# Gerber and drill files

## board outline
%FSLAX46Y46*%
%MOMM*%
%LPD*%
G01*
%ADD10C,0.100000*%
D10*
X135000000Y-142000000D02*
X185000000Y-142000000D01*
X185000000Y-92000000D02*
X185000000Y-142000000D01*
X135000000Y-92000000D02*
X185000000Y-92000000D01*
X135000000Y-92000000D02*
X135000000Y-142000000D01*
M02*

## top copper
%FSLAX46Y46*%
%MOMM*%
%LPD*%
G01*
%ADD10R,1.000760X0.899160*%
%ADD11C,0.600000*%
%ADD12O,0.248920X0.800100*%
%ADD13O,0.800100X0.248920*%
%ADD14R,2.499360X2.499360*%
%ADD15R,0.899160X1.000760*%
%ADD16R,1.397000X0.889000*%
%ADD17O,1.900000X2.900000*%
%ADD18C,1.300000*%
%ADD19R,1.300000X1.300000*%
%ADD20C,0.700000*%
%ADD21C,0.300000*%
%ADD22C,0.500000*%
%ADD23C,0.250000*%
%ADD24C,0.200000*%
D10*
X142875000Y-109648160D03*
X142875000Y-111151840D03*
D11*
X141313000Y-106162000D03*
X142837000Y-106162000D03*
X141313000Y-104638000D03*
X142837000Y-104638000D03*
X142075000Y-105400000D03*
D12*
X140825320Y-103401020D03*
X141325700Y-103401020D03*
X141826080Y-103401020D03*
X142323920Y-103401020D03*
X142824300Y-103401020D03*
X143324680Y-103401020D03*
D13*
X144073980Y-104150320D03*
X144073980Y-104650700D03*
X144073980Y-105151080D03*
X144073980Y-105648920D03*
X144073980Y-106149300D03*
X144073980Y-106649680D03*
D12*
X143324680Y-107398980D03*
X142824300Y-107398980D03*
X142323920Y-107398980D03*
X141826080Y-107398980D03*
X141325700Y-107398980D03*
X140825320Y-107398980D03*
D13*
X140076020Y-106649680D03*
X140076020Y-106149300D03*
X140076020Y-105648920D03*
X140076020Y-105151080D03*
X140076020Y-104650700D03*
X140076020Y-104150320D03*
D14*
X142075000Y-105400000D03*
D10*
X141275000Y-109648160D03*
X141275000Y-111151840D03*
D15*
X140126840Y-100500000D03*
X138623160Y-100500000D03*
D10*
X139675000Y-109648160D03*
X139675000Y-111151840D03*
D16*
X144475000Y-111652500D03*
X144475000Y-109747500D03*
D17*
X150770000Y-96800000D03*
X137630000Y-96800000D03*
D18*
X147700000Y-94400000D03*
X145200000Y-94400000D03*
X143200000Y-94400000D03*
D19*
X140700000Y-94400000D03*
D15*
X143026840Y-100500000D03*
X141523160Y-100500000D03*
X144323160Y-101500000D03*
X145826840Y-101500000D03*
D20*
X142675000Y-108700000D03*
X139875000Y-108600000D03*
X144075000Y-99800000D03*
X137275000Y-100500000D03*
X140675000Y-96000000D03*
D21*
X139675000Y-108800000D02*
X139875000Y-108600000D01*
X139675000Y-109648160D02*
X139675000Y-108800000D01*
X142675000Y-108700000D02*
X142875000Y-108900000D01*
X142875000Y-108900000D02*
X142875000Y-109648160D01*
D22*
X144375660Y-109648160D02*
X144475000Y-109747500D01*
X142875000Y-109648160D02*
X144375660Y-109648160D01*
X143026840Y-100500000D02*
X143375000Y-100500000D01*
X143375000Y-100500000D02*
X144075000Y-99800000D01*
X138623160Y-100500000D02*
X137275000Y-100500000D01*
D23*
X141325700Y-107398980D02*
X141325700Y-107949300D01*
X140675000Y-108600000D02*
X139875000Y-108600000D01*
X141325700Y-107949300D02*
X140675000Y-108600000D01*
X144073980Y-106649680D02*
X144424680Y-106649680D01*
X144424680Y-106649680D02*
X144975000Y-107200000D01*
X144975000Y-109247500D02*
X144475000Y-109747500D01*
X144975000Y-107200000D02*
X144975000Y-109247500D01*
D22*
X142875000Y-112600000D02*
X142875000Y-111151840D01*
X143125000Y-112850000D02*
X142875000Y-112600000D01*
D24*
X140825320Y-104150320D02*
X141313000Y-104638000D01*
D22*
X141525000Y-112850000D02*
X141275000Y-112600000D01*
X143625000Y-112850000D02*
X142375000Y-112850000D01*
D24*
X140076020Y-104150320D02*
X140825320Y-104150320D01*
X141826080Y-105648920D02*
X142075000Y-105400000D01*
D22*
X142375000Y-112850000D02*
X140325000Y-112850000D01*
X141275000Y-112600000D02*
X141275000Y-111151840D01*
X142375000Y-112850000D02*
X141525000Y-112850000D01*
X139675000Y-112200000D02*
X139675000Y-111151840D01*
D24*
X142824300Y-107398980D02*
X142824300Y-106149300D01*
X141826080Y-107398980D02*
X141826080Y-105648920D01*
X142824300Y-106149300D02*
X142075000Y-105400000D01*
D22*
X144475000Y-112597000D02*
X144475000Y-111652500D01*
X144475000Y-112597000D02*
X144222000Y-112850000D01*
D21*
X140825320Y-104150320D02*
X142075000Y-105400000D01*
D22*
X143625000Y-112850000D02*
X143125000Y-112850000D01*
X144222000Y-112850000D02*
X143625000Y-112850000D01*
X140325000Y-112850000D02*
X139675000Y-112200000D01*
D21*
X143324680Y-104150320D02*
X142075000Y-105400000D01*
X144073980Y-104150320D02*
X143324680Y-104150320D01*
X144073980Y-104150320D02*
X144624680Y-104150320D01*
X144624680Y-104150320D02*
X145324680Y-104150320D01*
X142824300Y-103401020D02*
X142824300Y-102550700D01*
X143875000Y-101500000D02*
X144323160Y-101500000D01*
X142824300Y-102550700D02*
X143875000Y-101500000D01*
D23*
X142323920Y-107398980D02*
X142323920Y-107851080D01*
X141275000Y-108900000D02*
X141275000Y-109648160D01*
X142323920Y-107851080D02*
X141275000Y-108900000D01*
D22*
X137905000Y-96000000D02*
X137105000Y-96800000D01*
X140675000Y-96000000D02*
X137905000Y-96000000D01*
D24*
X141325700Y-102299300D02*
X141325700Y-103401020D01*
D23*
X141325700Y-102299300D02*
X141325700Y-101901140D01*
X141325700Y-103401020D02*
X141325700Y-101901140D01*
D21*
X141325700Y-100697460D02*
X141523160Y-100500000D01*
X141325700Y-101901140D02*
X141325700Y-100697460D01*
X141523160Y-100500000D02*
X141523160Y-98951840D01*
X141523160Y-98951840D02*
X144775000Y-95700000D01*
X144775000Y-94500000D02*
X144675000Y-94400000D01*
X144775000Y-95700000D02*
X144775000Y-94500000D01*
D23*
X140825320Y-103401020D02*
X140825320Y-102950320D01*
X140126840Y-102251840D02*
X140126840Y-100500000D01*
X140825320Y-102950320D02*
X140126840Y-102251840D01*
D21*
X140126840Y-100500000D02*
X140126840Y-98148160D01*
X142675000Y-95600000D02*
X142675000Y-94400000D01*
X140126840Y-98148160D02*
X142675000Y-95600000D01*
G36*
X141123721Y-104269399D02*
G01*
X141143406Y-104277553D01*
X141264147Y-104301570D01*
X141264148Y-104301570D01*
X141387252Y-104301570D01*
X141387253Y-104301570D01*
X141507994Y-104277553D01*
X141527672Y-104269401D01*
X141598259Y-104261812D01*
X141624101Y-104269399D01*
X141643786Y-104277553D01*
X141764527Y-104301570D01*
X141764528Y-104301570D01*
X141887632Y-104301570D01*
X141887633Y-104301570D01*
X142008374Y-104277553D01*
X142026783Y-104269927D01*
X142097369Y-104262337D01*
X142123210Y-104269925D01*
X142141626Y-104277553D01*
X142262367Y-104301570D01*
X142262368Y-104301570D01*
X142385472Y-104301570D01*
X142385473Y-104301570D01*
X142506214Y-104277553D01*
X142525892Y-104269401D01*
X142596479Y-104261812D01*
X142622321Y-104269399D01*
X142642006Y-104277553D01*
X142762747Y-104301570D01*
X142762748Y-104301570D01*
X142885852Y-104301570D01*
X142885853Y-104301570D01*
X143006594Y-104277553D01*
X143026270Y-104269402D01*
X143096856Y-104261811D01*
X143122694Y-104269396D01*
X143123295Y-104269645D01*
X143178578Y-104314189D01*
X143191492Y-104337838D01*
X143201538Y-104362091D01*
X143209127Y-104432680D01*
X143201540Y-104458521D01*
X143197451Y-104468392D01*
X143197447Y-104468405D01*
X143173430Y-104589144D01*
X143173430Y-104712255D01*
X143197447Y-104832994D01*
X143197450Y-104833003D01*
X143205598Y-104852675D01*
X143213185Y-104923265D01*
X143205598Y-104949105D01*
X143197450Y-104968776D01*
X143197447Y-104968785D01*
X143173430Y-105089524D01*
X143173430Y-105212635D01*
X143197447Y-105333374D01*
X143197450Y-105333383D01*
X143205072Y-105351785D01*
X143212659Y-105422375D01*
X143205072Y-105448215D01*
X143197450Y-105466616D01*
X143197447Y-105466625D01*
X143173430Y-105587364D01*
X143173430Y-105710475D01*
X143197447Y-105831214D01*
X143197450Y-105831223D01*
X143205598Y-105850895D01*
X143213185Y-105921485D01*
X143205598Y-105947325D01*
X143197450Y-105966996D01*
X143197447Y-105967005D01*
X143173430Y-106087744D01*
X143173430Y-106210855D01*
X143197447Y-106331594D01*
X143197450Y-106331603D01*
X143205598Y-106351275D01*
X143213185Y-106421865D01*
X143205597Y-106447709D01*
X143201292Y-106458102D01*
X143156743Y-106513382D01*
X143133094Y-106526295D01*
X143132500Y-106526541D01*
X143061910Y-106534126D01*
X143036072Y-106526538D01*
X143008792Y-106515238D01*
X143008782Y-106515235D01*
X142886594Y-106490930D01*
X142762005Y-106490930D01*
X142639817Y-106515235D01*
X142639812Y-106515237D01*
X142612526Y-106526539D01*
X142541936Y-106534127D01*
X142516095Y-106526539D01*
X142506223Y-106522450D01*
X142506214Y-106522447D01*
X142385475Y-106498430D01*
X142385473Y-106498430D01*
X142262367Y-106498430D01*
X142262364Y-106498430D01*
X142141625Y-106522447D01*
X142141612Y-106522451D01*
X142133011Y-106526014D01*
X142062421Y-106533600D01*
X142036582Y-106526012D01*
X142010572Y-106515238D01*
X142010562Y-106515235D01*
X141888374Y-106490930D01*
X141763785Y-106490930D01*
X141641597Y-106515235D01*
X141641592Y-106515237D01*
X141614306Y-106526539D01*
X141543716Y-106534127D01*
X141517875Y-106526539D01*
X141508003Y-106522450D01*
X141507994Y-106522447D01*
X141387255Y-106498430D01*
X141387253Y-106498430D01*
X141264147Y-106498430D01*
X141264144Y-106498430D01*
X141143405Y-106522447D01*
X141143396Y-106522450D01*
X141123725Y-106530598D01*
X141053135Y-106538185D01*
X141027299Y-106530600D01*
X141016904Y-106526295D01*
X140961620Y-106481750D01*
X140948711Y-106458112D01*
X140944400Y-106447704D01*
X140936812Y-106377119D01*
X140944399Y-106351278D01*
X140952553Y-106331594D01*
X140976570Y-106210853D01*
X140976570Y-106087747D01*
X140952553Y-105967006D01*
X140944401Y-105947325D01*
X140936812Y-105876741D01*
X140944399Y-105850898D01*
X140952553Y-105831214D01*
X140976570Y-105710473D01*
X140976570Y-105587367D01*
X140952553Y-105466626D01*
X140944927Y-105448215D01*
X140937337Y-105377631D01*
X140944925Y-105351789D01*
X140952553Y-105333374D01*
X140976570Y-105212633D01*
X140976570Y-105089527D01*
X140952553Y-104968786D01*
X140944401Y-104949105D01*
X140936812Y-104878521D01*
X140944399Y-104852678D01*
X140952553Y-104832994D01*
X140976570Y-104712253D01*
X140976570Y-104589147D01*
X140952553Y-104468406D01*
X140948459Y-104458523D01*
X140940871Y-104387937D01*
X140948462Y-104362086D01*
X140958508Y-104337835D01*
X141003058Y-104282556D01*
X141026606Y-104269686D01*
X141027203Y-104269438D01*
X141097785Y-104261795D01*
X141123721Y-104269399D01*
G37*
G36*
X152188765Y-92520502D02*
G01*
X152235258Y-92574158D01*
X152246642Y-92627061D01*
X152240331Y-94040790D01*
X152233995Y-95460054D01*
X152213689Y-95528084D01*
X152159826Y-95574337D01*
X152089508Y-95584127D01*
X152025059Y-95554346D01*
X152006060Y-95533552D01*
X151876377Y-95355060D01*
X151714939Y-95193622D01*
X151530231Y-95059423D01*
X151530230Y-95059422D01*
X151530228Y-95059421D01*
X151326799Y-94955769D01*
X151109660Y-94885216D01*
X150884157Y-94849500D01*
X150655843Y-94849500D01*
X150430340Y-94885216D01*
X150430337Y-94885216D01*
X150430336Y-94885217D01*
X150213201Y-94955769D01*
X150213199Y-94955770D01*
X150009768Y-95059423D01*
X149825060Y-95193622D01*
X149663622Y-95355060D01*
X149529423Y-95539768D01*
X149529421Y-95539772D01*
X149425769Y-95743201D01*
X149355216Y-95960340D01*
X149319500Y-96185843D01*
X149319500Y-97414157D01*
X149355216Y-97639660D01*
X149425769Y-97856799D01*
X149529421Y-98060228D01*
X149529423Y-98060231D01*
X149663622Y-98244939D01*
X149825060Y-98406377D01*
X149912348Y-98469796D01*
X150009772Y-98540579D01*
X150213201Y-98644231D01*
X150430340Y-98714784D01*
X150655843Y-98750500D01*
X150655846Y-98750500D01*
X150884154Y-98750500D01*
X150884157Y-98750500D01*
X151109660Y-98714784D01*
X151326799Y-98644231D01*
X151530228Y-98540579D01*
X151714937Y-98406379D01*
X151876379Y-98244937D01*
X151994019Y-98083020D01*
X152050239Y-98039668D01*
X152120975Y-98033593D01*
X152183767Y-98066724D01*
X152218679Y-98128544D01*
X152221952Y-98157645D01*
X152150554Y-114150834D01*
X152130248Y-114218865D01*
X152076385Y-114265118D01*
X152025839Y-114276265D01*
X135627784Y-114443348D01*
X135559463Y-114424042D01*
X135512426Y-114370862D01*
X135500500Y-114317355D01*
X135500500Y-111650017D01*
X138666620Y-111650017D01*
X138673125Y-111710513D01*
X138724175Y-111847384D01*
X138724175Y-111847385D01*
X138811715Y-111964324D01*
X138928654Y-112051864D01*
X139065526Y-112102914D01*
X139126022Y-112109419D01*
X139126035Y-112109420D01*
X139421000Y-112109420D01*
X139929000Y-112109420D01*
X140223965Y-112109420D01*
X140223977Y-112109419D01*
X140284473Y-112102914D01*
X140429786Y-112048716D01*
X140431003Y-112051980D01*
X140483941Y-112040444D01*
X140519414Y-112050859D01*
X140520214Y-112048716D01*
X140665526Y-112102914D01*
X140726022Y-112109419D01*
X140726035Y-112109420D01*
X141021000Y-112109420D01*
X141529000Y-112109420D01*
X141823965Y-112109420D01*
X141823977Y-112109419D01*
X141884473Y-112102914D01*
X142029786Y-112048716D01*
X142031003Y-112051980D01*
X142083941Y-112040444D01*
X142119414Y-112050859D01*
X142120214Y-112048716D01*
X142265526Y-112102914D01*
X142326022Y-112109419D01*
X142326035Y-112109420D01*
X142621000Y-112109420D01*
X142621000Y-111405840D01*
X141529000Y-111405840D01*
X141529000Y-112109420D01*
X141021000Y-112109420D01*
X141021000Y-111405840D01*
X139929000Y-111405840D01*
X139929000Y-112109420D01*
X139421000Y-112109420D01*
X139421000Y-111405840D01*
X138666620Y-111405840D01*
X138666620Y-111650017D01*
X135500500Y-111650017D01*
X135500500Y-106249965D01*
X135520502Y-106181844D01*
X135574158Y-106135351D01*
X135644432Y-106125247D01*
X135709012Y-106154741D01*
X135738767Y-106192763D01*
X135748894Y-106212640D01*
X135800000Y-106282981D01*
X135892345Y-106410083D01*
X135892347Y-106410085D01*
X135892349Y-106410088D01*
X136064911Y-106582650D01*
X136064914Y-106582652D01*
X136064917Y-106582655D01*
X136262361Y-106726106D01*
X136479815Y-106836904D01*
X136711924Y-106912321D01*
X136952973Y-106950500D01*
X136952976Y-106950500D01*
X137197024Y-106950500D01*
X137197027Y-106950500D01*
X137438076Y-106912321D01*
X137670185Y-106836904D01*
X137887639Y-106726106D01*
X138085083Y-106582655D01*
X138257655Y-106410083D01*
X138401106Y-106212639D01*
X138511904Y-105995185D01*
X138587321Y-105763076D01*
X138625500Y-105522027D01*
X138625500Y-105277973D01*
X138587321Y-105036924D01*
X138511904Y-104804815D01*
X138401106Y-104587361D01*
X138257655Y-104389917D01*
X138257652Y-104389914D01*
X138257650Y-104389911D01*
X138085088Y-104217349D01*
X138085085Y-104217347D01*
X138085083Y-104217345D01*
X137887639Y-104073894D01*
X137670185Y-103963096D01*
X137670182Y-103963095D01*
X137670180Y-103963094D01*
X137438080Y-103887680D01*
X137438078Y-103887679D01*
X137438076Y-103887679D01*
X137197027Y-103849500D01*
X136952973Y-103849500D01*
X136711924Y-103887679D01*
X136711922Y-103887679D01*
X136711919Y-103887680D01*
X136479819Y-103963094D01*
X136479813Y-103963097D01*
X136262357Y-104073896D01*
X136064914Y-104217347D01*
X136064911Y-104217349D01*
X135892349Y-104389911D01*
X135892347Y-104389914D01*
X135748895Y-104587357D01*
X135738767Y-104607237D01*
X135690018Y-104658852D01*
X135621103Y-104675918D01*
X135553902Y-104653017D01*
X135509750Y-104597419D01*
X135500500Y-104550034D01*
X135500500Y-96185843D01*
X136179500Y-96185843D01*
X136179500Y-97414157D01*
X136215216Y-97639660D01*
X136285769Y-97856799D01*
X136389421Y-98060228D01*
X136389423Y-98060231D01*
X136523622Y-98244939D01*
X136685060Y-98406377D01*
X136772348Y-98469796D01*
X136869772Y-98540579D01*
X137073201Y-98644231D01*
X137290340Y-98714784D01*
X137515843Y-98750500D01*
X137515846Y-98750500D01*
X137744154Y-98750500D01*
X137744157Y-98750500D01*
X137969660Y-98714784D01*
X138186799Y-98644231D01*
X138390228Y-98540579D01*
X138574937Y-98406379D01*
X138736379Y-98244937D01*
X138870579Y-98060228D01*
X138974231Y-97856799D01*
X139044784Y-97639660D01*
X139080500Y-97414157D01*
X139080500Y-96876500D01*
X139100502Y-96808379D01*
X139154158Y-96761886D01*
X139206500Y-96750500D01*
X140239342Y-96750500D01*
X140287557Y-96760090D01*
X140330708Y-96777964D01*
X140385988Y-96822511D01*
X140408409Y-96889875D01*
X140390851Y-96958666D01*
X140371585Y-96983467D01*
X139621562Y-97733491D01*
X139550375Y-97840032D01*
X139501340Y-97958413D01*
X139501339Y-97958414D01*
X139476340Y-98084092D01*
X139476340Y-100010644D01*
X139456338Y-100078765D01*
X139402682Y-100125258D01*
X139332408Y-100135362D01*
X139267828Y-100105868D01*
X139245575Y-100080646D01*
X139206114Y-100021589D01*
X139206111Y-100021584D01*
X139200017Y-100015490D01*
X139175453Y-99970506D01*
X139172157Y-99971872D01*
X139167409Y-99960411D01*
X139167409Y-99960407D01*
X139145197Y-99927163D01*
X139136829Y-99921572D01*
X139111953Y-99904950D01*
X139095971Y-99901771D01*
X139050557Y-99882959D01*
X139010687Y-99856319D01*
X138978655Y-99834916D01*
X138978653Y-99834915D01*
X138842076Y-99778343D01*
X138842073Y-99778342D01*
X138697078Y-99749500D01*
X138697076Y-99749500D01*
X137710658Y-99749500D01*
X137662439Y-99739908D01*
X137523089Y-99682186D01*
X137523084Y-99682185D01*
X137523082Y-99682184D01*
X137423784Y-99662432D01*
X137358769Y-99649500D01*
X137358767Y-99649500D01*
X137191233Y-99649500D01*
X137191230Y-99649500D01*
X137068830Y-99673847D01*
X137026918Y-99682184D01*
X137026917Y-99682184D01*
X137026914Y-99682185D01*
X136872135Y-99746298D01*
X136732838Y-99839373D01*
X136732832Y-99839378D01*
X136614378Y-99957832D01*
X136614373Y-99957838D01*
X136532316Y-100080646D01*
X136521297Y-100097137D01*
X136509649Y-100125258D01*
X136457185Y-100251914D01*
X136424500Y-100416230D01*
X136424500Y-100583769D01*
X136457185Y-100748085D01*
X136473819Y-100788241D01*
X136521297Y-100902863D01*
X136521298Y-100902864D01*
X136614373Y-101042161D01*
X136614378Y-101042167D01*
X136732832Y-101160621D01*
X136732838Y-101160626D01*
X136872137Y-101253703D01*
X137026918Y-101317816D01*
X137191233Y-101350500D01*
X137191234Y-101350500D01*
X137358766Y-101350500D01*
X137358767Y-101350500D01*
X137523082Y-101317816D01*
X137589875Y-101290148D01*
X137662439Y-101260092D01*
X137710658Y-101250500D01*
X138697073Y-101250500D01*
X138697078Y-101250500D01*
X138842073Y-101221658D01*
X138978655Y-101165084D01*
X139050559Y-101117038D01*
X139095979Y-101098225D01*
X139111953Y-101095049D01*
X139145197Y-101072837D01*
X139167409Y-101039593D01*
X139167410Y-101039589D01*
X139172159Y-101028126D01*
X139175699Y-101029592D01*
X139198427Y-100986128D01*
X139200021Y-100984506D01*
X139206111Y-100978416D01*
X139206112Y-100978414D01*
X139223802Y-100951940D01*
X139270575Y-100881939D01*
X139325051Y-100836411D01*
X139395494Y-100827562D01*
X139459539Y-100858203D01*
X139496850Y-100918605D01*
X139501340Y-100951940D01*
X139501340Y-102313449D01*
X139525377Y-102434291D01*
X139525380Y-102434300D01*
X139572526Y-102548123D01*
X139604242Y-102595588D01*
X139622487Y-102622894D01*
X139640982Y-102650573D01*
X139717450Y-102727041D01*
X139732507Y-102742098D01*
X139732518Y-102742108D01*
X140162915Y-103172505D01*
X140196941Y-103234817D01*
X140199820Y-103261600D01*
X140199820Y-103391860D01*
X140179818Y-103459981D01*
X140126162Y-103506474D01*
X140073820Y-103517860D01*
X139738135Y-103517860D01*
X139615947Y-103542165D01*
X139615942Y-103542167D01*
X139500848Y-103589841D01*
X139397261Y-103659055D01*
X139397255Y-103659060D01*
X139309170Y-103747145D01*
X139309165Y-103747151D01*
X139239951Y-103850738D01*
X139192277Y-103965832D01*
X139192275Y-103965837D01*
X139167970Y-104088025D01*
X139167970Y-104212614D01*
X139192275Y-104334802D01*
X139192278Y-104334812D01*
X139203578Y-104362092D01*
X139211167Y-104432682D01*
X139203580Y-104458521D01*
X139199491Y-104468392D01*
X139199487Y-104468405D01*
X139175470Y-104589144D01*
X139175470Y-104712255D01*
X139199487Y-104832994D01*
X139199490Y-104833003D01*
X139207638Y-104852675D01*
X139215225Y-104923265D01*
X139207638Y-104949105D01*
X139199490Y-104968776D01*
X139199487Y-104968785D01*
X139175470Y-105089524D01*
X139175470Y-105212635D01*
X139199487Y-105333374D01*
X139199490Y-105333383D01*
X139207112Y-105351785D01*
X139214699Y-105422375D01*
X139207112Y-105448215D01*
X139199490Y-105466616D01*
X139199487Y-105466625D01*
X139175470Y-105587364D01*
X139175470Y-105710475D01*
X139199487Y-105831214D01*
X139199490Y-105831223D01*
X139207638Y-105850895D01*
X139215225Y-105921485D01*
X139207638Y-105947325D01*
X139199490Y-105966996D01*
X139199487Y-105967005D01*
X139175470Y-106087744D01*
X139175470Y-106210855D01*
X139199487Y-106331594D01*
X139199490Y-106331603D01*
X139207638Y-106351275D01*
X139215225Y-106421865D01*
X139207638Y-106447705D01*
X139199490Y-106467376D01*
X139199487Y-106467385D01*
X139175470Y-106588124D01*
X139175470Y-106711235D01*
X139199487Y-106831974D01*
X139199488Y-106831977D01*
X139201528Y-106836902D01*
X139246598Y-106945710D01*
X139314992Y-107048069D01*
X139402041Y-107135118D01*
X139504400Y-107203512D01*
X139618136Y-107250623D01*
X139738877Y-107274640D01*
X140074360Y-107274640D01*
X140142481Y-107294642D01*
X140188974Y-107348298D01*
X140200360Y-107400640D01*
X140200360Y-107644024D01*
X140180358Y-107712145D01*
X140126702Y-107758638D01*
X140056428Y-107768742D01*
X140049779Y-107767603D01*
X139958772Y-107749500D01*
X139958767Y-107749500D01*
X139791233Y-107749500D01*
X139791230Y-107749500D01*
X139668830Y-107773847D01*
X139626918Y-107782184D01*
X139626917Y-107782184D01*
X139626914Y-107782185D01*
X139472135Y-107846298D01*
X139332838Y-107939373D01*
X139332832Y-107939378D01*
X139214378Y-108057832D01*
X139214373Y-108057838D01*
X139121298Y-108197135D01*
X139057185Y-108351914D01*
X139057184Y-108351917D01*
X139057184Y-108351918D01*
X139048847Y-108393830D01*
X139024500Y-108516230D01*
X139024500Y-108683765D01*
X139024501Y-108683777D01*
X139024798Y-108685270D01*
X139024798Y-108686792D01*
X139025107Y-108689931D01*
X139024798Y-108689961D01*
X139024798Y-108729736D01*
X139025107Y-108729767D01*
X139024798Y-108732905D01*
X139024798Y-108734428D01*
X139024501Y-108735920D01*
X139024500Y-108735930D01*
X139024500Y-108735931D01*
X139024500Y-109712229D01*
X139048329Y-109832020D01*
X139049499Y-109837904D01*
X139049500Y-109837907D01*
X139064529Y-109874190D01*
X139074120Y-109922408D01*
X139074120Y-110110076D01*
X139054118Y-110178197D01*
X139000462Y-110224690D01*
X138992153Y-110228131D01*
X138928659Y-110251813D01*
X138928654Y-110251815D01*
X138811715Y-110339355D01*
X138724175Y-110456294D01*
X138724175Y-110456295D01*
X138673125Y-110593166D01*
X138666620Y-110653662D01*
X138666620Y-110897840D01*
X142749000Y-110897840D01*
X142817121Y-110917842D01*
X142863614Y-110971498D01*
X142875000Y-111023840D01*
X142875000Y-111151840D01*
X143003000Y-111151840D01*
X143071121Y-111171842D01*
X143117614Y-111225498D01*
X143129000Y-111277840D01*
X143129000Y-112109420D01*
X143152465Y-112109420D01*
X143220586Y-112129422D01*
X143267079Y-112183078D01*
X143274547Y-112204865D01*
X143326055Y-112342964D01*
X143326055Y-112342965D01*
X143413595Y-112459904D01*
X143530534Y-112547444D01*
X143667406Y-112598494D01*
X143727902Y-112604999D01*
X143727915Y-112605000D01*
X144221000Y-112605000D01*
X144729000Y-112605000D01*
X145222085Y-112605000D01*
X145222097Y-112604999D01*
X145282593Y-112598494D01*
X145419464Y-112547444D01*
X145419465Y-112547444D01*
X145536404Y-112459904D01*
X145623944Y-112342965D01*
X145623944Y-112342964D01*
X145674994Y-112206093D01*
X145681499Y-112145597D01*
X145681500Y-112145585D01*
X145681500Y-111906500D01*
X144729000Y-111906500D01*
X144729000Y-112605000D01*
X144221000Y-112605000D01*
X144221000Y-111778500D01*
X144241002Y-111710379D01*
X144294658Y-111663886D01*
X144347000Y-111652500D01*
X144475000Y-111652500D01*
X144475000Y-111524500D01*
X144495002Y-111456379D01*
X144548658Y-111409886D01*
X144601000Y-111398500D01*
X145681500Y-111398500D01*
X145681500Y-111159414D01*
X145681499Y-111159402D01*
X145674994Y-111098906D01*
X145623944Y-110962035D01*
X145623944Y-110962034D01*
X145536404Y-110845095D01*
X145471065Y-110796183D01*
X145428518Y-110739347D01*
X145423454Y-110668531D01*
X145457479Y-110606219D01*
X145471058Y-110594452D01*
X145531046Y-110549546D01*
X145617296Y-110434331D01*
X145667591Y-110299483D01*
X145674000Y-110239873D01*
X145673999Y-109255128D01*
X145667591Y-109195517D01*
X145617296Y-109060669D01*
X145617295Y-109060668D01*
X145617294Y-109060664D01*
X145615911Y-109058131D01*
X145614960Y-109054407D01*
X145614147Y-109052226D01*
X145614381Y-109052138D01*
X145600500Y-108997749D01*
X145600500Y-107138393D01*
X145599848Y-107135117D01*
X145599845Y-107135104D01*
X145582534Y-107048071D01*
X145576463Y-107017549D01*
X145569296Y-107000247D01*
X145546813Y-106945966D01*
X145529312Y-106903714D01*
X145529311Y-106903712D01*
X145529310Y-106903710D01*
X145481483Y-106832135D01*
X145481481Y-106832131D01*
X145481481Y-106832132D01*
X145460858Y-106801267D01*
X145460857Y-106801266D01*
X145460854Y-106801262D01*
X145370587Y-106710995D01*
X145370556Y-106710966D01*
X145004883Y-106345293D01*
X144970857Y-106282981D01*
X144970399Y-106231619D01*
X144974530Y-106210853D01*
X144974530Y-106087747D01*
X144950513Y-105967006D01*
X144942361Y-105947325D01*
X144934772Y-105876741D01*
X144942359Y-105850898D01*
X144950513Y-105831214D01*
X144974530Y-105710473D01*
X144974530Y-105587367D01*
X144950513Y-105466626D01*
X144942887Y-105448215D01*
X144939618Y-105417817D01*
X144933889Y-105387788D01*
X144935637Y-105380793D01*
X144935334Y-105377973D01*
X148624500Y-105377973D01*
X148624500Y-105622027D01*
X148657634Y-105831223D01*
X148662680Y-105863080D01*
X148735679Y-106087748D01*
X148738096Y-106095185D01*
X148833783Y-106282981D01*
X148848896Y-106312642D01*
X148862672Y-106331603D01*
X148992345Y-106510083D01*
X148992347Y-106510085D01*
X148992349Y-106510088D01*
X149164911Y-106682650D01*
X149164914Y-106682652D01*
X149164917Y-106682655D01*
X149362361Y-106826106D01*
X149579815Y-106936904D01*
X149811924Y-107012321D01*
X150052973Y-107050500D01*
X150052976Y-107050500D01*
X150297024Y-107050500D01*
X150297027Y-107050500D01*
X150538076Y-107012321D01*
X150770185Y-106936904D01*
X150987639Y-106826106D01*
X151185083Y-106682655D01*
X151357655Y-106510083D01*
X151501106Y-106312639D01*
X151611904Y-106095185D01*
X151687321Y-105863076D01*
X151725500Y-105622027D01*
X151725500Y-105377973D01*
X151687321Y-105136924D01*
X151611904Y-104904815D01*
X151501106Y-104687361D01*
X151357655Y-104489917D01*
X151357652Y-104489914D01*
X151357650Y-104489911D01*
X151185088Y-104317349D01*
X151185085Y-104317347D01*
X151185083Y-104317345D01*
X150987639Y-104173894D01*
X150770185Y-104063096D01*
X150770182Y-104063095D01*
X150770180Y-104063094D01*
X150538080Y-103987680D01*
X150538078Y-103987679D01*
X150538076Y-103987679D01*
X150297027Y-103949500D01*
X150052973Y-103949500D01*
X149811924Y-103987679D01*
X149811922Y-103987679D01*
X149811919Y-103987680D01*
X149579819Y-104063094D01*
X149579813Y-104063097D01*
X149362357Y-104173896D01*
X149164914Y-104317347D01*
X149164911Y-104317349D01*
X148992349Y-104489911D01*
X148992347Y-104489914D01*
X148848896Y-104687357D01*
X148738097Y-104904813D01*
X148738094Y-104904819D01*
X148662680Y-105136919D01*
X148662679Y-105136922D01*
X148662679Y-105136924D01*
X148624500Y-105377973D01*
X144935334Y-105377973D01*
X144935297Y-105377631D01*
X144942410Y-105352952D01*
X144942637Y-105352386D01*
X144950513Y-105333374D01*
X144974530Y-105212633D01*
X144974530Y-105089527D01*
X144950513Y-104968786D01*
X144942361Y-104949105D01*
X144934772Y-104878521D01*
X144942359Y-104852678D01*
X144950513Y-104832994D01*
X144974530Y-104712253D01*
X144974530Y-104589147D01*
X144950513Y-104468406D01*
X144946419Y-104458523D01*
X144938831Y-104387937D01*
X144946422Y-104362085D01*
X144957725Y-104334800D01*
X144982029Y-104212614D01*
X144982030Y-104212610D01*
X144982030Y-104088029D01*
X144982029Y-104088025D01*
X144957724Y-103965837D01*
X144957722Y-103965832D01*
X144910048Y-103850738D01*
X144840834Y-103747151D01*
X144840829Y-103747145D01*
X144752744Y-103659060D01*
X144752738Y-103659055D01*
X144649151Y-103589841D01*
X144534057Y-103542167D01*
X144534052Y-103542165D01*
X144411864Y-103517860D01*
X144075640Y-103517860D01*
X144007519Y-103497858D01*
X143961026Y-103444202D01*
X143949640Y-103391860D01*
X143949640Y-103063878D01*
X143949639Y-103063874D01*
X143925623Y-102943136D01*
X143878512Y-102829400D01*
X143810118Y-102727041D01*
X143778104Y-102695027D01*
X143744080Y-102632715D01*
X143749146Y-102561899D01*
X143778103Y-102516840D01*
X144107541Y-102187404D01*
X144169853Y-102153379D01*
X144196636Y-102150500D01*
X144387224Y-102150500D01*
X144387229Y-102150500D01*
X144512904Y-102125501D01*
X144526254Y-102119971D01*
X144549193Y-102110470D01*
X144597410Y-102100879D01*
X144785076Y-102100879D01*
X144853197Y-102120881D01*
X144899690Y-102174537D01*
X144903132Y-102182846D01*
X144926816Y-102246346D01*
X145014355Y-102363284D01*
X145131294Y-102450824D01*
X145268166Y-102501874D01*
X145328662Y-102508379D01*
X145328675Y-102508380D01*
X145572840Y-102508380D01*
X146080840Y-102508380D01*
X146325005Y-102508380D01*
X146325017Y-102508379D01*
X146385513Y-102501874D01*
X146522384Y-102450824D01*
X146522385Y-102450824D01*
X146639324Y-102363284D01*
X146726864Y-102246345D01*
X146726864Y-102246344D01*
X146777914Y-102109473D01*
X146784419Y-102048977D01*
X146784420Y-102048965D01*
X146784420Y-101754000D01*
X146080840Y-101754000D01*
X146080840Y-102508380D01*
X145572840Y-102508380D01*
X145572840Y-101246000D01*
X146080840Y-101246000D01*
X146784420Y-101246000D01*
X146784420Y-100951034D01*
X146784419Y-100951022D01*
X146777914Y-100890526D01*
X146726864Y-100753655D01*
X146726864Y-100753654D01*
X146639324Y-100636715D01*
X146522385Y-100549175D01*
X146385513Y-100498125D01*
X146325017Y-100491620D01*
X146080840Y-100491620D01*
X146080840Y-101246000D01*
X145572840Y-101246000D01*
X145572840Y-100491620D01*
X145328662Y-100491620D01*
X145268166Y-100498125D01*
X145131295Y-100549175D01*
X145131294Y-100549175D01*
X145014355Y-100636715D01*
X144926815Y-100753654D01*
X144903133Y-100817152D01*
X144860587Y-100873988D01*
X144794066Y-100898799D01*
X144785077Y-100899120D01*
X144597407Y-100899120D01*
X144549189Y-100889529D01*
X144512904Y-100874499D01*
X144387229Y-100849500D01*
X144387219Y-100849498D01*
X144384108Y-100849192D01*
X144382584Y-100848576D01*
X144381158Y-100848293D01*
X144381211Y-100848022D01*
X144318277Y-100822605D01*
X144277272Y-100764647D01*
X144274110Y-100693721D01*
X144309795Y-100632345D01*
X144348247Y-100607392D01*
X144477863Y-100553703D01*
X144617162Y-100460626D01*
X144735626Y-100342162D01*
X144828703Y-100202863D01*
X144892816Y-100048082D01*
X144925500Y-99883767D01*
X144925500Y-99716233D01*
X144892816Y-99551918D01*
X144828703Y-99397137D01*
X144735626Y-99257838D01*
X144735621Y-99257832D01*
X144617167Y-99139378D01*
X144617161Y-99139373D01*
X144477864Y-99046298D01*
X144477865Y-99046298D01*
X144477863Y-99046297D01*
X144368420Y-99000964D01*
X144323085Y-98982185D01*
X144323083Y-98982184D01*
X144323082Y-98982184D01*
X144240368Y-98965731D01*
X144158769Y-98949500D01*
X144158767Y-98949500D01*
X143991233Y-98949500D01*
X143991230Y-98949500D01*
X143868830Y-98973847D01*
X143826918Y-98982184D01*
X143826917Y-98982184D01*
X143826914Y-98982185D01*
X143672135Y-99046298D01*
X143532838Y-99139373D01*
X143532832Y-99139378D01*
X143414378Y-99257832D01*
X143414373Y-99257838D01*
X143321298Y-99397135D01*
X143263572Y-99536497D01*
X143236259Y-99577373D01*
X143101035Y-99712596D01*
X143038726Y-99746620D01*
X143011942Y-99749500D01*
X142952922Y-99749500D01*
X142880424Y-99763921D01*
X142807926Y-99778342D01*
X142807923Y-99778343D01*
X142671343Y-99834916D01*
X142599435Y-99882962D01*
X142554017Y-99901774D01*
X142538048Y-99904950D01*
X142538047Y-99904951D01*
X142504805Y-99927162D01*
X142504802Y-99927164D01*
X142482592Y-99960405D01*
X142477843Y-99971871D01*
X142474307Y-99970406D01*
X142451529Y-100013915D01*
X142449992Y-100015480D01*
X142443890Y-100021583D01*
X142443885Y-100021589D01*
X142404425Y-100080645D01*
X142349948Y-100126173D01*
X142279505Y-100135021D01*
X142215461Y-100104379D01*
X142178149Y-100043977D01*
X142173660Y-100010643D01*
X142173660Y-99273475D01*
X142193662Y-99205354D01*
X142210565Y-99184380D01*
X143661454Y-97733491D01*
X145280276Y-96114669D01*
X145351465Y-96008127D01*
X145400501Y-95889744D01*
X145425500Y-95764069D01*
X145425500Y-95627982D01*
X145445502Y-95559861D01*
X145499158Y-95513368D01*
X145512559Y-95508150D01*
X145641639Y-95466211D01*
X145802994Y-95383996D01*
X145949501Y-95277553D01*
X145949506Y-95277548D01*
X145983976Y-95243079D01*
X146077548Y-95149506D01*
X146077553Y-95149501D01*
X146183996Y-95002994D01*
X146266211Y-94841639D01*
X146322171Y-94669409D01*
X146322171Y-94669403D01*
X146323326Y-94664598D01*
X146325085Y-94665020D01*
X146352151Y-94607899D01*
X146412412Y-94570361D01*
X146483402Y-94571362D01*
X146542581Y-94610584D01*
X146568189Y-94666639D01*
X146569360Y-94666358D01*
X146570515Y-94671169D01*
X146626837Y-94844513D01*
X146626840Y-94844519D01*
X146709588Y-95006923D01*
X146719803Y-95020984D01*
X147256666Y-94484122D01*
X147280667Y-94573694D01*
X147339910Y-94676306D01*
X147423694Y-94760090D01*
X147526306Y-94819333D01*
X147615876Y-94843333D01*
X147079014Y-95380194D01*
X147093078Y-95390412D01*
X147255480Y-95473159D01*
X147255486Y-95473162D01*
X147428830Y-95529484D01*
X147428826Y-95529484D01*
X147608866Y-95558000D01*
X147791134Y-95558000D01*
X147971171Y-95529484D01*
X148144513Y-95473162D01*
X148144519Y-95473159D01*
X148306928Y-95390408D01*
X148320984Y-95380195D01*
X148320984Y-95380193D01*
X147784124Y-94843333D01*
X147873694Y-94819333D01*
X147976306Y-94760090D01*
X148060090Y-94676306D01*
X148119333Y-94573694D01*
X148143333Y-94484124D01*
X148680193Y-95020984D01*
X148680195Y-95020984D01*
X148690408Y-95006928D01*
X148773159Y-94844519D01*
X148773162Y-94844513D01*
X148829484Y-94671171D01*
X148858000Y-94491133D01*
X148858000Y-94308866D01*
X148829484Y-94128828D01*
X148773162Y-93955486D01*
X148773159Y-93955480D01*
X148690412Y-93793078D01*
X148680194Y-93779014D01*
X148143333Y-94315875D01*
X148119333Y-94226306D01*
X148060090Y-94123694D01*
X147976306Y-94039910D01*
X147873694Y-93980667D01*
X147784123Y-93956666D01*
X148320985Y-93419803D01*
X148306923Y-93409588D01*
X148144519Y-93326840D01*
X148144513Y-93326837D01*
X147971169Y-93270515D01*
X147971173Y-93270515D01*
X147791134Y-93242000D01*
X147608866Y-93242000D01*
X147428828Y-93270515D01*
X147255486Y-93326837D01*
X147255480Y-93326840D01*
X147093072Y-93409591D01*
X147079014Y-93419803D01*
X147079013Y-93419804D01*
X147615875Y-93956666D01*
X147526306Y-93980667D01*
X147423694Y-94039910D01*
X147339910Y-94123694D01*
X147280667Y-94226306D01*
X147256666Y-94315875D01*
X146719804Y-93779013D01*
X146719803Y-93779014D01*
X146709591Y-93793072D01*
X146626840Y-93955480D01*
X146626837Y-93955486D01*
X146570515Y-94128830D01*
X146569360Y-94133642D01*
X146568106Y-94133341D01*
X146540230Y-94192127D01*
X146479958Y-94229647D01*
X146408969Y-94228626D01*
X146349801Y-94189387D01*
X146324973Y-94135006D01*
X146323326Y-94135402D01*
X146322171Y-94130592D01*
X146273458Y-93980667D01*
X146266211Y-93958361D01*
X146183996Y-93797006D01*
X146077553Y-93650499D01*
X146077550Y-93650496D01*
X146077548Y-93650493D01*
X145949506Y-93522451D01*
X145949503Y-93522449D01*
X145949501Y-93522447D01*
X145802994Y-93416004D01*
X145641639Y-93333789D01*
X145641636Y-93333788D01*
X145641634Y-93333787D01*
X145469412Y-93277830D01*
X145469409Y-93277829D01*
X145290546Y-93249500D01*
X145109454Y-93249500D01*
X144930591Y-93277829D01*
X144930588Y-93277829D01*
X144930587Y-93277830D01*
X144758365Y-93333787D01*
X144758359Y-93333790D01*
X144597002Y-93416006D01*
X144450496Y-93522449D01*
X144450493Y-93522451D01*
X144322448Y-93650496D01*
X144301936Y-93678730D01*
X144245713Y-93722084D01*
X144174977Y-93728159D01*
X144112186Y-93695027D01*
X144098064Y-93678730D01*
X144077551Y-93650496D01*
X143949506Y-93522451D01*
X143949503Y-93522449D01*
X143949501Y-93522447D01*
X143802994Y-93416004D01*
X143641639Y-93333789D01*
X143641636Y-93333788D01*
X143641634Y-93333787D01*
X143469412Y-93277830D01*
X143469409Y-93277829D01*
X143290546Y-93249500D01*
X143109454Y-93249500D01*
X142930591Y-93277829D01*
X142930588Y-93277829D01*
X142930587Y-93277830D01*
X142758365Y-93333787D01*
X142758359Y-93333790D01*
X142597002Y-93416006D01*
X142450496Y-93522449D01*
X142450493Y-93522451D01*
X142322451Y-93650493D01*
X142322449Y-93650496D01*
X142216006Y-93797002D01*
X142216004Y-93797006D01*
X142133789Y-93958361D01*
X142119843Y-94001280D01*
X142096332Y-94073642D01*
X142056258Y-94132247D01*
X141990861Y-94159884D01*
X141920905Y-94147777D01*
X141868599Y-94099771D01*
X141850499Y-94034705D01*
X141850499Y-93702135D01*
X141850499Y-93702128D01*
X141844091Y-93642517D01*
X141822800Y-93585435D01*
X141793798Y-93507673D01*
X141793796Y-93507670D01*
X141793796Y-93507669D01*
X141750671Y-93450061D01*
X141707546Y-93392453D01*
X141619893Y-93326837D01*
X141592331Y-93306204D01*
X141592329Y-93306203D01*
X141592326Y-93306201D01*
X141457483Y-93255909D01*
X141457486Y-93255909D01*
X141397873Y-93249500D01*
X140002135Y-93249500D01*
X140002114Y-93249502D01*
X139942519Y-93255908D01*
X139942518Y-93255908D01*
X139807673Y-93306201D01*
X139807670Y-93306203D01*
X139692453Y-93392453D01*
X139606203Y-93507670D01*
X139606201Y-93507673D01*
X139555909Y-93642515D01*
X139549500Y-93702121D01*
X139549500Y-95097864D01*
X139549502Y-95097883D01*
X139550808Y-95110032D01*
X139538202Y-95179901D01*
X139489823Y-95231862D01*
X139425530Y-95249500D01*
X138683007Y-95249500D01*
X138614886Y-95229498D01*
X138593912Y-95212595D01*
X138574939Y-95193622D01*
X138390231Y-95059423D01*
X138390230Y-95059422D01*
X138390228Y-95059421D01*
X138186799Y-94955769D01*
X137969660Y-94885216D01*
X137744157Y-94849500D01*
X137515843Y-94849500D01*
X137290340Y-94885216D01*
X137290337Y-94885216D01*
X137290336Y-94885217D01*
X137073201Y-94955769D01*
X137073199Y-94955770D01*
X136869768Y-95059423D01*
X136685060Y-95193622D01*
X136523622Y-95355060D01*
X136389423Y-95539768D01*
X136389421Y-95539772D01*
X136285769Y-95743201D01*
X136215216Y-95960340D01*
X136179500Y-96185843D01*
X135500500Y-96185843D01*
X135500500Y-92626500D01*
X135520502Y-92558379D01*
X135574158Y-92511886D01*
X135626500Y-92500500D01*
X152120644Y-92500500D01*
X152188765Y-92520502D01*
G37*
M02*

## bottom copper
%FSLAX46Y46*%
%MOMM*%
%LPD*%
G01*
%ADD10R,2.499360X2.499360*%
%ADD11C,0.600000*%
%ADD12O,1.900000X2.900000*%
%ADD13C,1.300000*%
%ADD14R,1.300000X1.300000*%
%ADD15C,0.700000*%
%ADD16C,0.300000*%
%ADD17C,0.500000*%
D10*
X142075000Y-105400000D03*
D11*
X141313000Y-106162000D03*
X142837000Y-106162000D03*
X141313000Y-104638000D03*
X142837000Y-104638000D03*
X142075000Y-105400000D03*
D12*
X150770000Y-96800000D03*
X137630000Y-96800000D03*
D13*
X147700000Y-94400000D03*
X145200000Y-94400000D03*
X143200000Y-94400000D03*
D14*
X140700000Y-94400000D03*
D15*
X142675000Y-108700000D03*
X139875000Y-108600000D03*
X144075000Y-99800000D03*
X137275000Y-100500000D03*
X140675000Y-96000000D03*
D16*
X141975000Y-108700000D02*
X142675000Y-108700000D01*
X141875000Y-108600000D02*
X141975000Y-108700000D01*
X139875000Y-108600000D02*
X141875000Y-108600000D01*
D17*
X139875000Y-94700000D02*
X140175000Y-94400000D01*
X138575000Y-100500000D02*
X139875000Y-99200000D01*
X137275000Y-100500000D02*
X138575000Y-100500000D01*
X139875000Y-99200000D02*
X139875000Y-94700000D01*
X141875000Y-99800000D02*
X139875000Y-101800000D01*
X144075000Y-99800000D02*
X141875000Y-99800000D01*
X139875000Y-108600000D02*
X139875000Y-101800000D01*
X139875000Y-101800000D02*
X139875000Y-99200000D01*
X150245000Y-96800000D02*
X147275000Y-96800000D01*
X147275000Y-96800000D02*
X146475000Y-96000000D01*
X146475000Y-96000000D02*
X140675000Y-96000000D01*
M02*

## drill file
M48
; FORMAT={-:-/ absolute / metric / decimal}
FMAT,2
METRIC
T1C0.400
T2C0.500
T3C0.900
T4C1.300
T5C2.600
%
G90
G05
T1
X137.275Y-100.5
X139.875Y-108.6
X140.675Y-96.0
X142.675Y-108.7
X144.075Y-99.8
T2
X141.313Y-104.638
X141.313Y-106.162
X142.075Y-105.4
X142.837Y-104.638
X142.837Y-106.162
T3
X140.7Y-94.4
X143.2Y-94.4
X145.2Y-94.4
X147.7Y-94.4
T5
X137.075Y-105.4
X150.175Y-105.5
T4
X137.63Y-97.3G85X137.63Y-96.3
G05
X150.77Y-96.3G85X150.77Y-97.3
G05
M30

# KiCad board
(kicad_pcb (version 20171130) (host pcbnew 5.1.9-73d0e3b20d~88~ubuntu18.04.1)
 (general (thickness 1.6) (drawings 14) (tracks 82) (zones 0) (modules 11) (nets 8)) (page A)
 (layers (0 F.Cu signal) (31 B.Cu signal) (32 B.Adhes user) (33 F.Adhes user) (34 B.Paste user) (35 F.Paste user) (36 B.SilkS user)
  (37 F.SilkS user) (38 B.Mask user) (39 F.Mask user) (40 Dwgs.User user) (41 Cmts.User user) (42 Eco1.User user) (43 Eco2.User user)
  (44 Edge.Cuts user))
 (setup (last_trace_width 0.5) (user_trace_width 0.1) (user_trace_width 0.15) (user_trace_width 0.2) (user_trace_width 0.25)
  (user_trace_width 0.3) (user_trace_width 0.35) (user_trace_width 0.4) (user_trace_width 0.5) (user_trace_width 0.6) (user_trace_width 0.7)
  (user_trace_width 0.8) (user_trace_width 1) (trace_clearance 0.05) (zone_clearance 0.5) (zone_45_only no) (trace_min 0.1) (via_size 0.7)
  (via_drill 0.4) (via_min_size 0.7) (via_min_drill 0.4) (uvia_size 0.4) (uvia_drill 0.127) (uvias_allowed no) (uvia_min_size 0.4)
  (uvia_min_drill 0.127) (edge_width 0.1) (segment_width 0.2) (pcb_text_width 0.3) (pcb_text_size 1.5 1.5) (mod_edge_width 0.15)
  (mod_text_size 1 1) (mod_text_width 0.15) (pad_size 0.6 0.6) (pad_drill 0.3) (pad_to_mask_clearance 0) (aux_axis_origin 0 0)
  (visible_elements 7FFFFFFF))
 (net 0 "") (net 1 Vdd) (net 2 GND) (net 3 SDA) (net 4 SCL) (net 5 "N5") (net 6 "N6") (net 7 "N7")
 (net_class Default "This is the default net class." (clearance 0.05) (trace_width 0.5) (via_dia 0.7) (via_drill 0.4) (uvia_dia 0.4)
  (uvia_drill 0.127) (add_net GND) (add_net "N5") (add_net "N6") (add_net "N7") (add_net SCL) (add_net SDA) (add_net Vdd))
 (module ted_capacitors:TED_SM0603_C (layer F.Cu) (at 142.875 110.4 270)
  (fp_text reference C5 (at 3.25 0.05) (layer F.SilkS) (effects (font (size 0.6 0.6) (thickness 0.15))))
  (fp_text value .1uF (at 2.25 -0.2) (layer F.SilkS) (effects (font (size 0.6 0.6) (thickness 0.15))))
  (pad 1 smd rect (at -0.75184 0 270) (size 0.89916 1.00076) (layers F.Cu F.Paste F.Mask) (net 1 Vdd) (clearance 0.1))
  (pad 2 smd rect (at 0.75184 0 270) (size 0.89916 1.00076) (layers F.Cu F.Paste F.Mask) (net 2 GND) (clearance 0.1)))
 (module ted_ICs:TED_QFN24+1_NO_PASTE (layer F.Cu) (at 142.075 105.4)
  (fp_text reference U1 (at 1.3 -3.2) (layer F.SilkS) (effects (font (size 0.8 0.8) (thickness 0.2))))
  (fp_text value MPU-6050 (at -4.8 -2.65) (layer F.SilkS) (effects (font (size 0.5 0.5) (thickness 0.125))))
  (pad 25 smd rect (at 0 0 270) (size 2.49936 2.49936) (layers B.Cu B.Mask) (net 2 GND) (zone_connect 2))
  (pad 25 thru_hole circle (at -0.762 0.762 270) (size 0.6 0.6) (drill 0.5) (layers *.Cu) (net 2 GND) (zone_connect 2))
  (pad 25 thru_hole circle (at 0.762 0.762 270) (size 0.6 0.6) (drill 0.5) (layers *.Cu) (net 2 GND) (zone_connect 2))
  (pad 25 thru_hole circle (at -0.762 -0.762 270) (size 0.6 0.6) (drill 0.5) (layers *.Cu) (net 2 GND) (zone_connect 2))
  (pad 25 thru_hole circle (at 0.762 -0.762 270) (size 0.6 0.6) (drill 0.5) (layers *.Cu) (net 2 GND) (zone_connect 2))
  (pad 25 thru_hole circle (at 0 0 270) (size 0.6 0.6) (drill 0.5) (layers *.Cu) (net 2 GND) (zone_connect 2))
  (pad 24 smd oval (at -1.24968 -1.99898 270) (size 0.8001 0.24892) (layers F.Cu F.Paste F.Mask) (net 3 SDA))
  (pad 23 smd oval (at -0.7493 -1.99898 270) (size 0.8001 0.24892) (layers F.Cu F.Paste F.Mask) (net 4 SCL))
  (pad 22 smd oval (at -0.24892 -1.99898 270) (size 0.8001 0.24892) (layers F.Cu F.Paste F.Mask))
  (pad 21 smd oval (at 0.24892 -1.99898 270) (size 0.8001 0.24892) (layers F.Cu F.Paste F.Mask))
  (pad 20 smd oval (at 0.7493 -1.99898 270) (size 0.8001 0.24892) (layers F.Cu F.Paste F.Mask) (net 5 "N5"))
  (pad 19 smd oval (at 1.24968 -1.99898 270) (size 0.8001 0.24892) (layers F.Cu F.Paste F.Mask))
  (pad 18 smd oval (at 1.99898 -1.24968 180) (size 0.8001 0.24892) (layers F.Cu F.Paste F.Mask) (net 2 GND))
  (pad 17 smd oval (at 1.99898 -0.7493 180) (size 0.8001 0.24892) (layers F.Cu F.Paste F.Mask))
  (pad 16 smd oval (at 1.99898 -0.24892 180) (size 0.8001 0.24892) (layers F.Cu F.Paste F.Mask))
  (pad 15 smd oval (at 1.99898 0.24892 180) (size 0.8001 0.24892) (layers F.Cu F.Paste F.Mask))
  (pad 14 smd oval (at 1.99898 0.7493 180) (size 0.8001 0.24892) (layers F.Cu F.Paste F.Mask))
  (pad 13 smd oval (at 1.99898 1.24968 180) (size 0.8001 0.24892) (layers F.Cu F.Paste F.Mask) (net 1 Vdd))
  (pad 12 smd oval (at 1.24968 1.99898 90) (size 0.8001 0.24892) (layers F.Cu F.Paste F.Mask))
  (pad 11 smd oval (at 0.7493 1.99898 90) (size 0.8001 0.24892) (layers F.Cu F.Paste F.Mask) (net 2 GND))
  (pad 10 smd oval (at 0.24892 1.99898 90) (size 0.8001 0.24892) (layers F.Cu F.Paste F.Mask) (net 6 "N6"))
  (pad 9 smd oval (at -0.24892 1.99898 90) (size 0.8001 0.24892) (layers F.Cu F.Paste F.Mask) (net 2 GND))
  (pad 8 smd oval (at -0.7493 1.99898 90) (size 0.8001 0.24892) (layers F.Cu F.Paste F.Mask) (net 1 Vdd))
  (pad 7 smd oval (at -1.24968 1.99898 90) (size 0.8001 0.24892) (layers F.Cu F.Paste F.Mask))
  (pad 6 smd oval (at -1.99898 1.24968) (size 0.8001 0.24892) (layers F.Cu F.Paste F.Mask))
  (pad 5 smd oval (at -1.99898 0.7493) (size 0.8001 0.24892) (layers F.Cu F.Paste F.Mask))
  (pad 4 smd oval (at -1.99898 0.24892) (size 0.8001 0.24892) (layers F.Cu F.Paste F.Mask))
  (pad 3 smd oval (at -1.99898 -0.24892) (size 0.8001 0.24892) (layers F.Cu F.Paste F.Mask))
  (pad 2 smd oval (at -1.99898 -0.7493) (size 0.8001 0.24892) (layers F.Cu F.Paste F.Mask))
  (pad 1 smd oval (at -1.99898 -1.24968) (size 0.8001 0.24892) (layers F.Cu F.Paste F.Mask) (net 2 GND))
  (pad 25 smd rect (at 0 0 270) (size 2.49936 2.49936) (layers F.Cu F.Mask) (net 2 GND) (zone_connect 2)))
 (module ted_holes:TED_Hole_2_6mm (layer F.Cu) (at 150.175 105.5)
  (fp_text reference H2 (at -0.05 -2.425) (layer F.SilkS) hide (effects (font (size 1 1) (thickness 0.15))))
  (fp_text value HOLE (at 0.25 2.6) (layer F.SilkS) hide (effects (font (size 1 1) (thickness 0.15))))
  (pad "" np_thru_hole circle (at 0 0) (size 2.6 2.6) (drill 2.6) (layers *.Cu *.Mask F.SilkS)))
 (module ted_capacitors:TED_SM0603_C (layer F.Cu) (at 141.275 110.4 270)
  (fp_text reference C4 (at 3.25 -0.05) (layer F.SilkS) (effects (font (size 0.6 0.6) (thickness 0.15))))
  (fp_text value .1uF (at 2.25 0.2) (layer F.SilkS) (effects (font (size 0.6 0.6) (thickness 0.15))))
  (pad 1 smd rect (at -0.75184 0 270) (size 0.89916 1.00076) (layers F.Cu F.Paste F.Mask) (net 6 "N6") (clearance 0.1))
  (pad 2 smd rect (at 0.75184 0 270) (size 0.89916 1.00076) (layers F.Cu F.Paste F.Mask) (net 2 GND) (clearance 0.1)))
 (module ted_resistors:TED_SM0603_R (layer F.Cu) (at 139.375 100.5)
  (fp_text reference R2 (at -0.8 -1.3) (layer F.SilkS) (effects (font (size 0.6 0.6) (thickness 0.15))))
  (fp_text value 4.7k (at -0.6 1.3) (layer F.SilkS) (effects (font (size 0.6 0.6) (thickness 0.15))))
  (pad 2 smd rect (at 0.75184 0) (size 0.89916 1.00076) (layers F.Cu F.Paste F.Mask) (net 3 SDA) (clearance 0.1))
  (pad 1 smd rect (at -0.75184 0) (size 0.89916 1.00076) (layers F.Cu F.Paste F.Mask) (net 1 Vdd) (clearance 0.1)))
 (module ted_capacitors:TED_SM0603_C (layer F.Cu) (at 139.675 110.4 270)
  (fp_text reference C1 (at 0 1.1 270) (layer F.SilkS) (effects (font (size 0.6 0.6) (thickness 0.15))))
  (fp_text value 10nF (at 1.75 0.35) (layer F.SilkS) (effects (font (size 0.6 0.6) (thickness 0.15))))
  (pad 1 smd rect (at -0.75184 0 270) (size 0.89916 1.00076) (layers F.Cu F.Paste F.Mask) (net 1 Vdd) (clearance 0.1))
  (pad 2 smd rect (at 0.75184 0 270) (size 0.89916 1.00076) (layers F.Cu F.Paste F.Mask) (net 2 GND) (clearance 0.1)))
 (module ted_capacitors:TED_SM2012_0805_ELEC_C (layer F.Cu) (at 144.475 110.7 270)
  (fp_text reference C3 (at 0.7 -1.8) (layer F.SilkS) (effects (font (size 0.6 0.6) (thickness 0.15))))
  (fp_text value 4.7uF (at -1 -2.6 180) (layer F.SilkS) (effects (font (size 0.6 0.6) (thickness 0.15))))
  (pad 2 smd rect (at 0.9525 0 270) (size 0.889 1.397) (layers F.Cu F.Paste F.Mask) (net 2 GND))
  (pad 1 smd rect (at -0.9525 0 270) (size 0.889 1.397) (layers F.Cu F.Paste F.Mask) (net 1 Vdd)))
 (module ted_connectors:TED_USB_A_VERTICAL (layer F.Cu) (at 144.2 95.4)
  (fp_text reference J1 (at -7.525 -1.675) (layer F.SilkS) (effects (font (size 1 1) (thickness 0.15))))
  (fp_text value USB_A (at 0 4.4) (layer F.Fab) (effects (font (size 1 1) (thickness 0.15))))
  (pad 5 thru_hole oval (at 6.57 1.4) (size 1.9 2.9) (drill oval 1.3 2.3) (layers *.Cu *.Mask) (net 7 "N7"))
  (pad 5 thru_hole oval (at -6.57 1.4 180) (size 1.9 2.9) (drill oval 1.3 2.3) (layers *.Cu *.Mask) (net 7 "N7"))
  (pad 4 thru_hole circle (at 3.5 -1) (size 1.3 1.3) (drill 0.9) (layers *.Cu *.Mask) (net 2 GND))
  (pad 3 thru_hole circle (at 1 -1) (size 1.3 1.3) (drill 0.9) (layers *.Cu *.Mask) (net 4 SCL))
  (pad 2 thru_hole circle (at -1 -1) (size 1.3 1.3) (drill 0.9) (layers *.Cu *.Mask) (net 3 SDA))
  (pad 1 thru_hole rect (at -3.5 -1) (size 1.3 1.3) (drill 0.9) (layers *.Cu *.Mask) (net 1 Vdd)))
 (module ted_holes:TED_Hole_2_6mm (layer F.Cu) (at 137.075 105.4)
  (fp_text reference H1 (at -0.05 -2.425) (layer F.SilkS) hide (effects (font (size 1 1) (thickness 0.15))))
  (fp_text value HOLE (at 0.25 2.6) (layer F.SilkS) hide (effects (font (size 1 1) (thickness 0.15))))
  (pad "" np_thru_hole circle (at 0 0) (size 2.6 2.6) (drill 2.6) (layers *.Cu *.Mask F.SilkS)))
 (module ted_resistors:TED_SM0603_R (layer F.Cu) (at 142.275 100.5 180)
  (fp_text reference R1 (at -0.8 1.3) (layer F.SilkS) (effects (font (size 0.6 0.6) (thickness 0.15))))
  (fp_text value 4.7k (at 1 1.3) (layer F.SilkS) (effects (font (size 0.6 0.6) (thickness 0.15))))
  (pad 1 smd rect (at -0.75184 0 180) (size 0.89916 1.00076) (layers F.Cu F.Paste F.Mask) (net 1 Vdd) (clearance 0.1))
  (pad 2 smd rect (at 0.75184 0 180) (size 0.89916 1.00076) (layers F.Cu F.Paste F.Mask) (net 4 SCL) (clearance 0.1)))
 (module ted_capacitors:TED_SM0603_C (layer F.Cu) (at 145.075 101.5)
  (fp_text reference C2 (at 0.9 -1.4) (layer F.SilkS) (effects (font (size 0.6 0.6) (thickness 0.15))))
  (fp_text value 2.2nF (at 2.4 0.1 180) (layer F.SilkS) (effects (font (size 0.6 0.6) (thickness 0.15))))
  (pad 1 smd rect (at -0.75184 0) (size 0.89916 1.00076) (layers F.Cu F.Paste F.Mask) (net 5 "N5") (clearance 0.1))
  (pad 2 smd rect (at 0.75184 0) (size 0.89916 1.00076) (layers F.Cu F.Paste F.Mask) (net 2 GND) (clearance 0.1)))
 (gr_line (start 135 142) (end 185 142) (angle 90) (layer Edge.Cuts) (width 0.1))
 (gr_line (start 185 92) (end 185 142) (angle 90) (layer Edge.Cuts) (width 0.1))
 (gr_line (start 135 92) (end 185 92) (angle 90) (layer Edge.Cuts) (width 0.1))
 (gr_line (start 135 92) (end 135 142) (angle 90) (layer Edge.Cuts) (width 0.1))
 (segment (start 139.675 108.8) (end 139.875 108.6) (width 0.3) (layer F.Cu) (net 1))
 (segment (start 139.675 109.64816) (end 139.675 108.8) (width 0.3) (layer F.Cu) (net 1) (status 10))
 (segment (start 141.975 108.7) (end 142.675 108.7) (width 0.3) (layer B.Cu) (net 1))
 (via (at 142.675 108.7) (size 0.7) (drill 0.4) (layers F.Cu B.Cu) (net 1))
 (segment (start 141.875 108.6) (end 141.975 108.7) (width 0.3) (layer B.Cu) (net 1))
 (segment (start 139.875 108.6) (end 141.875 108.6) (width 0.3) (layer B.Cu) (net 1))
 (segment (start 142.675 108.7) (end 142.875 108.9) (width 0.3) (layer F.Cu) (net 1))
 (segment (start 142.875 108.9) (end 142.875 109.64816) (width 0.3) (layer F.Cu) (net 1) (status 20))
 (via (at 139.875 108.6) (size 0.7) (drill 0.4) (layers F.Cu B.Cu) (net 1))
 (segment (start 144.37566 109.64816) (end 144.475 109.7475) (width 0.5) (layer F.Cu) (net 1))
 (segment (start 142.875 109.64816) (end 144.37566 109.64816) (width 0.5) (layer F.Cu) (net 1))
 (segment (start 139.875 94.7) (end 140.175 94.4) (width 0.5) (layer B.Cu) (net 1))
 (segment (start 143.02684 100.5) (end 143.375 100.5) (width 0.5) (layer F.Cu) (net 1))
 (via (at 144.075 99.8) (size 0.7) (drill 0.4) (layers F.Cu B.Cu) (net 1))
 (segment (start 143.375 100.5) (end 144.075 99.8) (width 0.5) (layer F.Cu) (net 1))
 (via (at 137.275 100.5) (size 0.7) (drill 0.4) (layers F.Cu B.Cu) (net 1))
 (segment (start 138.62316 100.5) (end 137.275 100.5) (width 0.5) (layer F.Cu) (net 1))
 (segment (start 138.575 100.5) (end 139.875 99.2) (width 0.5) (layer B.Cu) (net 1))
 (segment (start 137.275 100.5) (end 138.575 100.5) (width 0.5) (layer B.Cu) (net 1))
 (segment (start 139.875 99.2) (end 139.875 94.7) (width 0.5) (layer B.Cu) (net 1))
 (segment (start 141.875 99.8) (end 139.875 101.8) (width 0.5) (layer B.Cu) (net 1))
 (segment (start 144.075 99.8) (end 141.875 99.8) (width 0.5) (layer B.Cu) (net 1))
 (segment (start 139.875 108.6) (end 139.875 101.8) (width 0.5) (layer B.Cu) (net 1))
 (segment (start 139.875 101.8) (end 139.875 99.2) (width 0.5) (layer B.Cu) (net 1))
 (segment (start 141.3257 107.39898) (end 141.3257 107.9493) (width 0.25) (layer F.Cu) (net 1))
 (segment (start 140.675 108.6) (end 139.875 108.6) (width 0.25) (layer F.Cu) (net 1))
 (segment (start 141.3257 107.9493) (end 140.675 108.6) (width 0.25) (layer F.Cu) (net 1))
 (segment (start 144.07398 106.64968) (end 144.42468 106.64968) (width 0.25) (layer F.Cu) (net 1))
 (segment (start 144.42468 106.64968) (end 144.975 107.2) (width 0.25) (layer F.Cu) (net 1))
 (segment (start 144.975 109.2475) (end 144.475 109.7475) (width 0.25) (layer F.Cu) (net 1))
 (segment (start 144.975 107.2) (end 144.975 109.2475) (width 0.25) (layer F.Cu) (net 1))
 (segment (start 142.875 112.6) (end 142.875 111.15184) (width 0.5) (layer F.Cu) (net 2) (status 20))
 (segment (start 143.125 112.85) (end 142.875 112.6) (width 0.5) (layer F.Cu) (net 2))
 (segment (start 140.82532 104.15032) (end 141.313 104.638) (width 0.2) (layer F.Cu) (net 2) (status 30))
 (segment (start 141.525 112.85) (end 141.275 112.6) (width 0.5) (layer F.Cu) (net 2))
 (segment (start 143.625 112.85) (end 142.375 112.85) (width 0.5) (layer F.Cu) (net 2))
 (segment (start 140.07602 104.15032) (end 140.82532 104.15032) (width 0.2) (layer F.Cu) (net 2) (status 30))
 (segment (start 141.82608 105.64892) (end 142.075 105.4) (width 0.2) (layer F.Cu) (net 2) (status 30))
 (segment (start 142.375 112.85) (end 140.325 112.85) (width 0.5) (layer F.Cu) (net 2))
 (segment (start 141.275 112.6) (end 141.275 111.15184) (width 0.5) (layer F.Cu) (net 2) (status 20))
 (segment (start 142.375 112.85) (end 141.525 112.85) (width 0.5) (layer F.Cu) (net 2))
 (segment (start 139.675 112.2) (end 139.675 111.15184) (width 0.5) (layer F.Cu) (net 2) (status 20))
 (segment (start 142.8243 107.39898) (end 142.8243 106.1493) (width 0.2) (layer F.Cu) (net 2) (status 30))
 (segment (start 141.82608 107.39898) (end 141.82608 105.64892) (width 0.2) (layer F.Cu) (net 2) (status 30))
 (segment (start 142.8243 106.1493) (end 142.075 105.4) (width 0.2) (layer F.Cu) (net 2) (status 30))
 (segment (start 144.475 112.597) (end 144.475 111.6525) (width 0.5) (layer F.Cu) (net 2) (status 20))
 (segment (start 144.475 112.597) (end 144.222 112.85) (width 0.5) (layer F.Cu) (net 2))
 (segment (start 140.82532 104.15032) (end 142.075 105.4) (width 0.3) (layer F.Cu) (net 2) (status 30))
 (segment (start 143.625 112.85) (end 143.125 112.85) (width 0.5) (layer F.Cu) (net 2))
 (segment (start 144.222 112.85) (end 143.625 112.85) (width 0.5) (layer F.Cu) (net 2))
 (segment (start 140.325 112.85) (end 139.675 112.2) (width 0.5) (layer F.Cu) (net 2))
 (segment (start 143.32468 104.15032) (end 142.075 105.4) (width 0.3) (layer F.Cu) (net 2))
 (segment (start 144.07398 104.15032) (end 143.32468 104.15032) (width 0.3) (layer F.Cu) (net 2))
 (segment (start 144.07398 104.15032) (end 144.62468 104.15032) (width 0.3) (layer F.Cu) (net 2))
 (segment (start 144.62468 104.15032) (end 145.32468 104.15032) (width 0.3) (layer F.Cu) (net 2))
 (segment (start 142.8243 103.40102) (end 142.8243 102.5507) (width 0.3) (layer F.Cu) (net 5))
 (segment (start 143.875 101.5) (end 144.32316 101.5) (width 0.3) (layer F.Cu) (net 5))
 (segment (start 142.8243 102.5507) (end 143.875 101.5) (width 0.3) (layer F.Cu) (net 5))
 (segment (start 142.32392 107.39898) (end 142.32392 107.85108) (width 0.25) (layer F.Cu) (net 6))
 (segment (start 141.275 108.9) (end 141.275 109.64816) (width 0.25) (layer F.Cu) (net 6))
 (segment (start 142.32392 107.85108) (end 141.275 108.9) (width 0.25) (layer F.Cu) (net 6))
 (segment (start 150.245 96.8) (end 147.275 96.8) (width 0.5) (layer B.Cu) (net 7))
 (via (at 140.675 96) (size 0.7) (drill 0.4) (layers F.Cu B.Cu) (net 7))
 (segment (start 147.275 96.8) (end 146.475 96) (width 0.5) (layer B.Cu) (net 7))
 (segment (start 146.475 96) (end 140.675 96) (width 0.5) (layer B.Cu) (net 7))
 (segment (start 137.905 96) (end 137.105 96.8) (width 0.5) (layer F.Cu) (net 7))
 (segment (start 140.675 96) (end 137.905 96) (width 0.5) (layer F.Cu) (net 7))
 (segment (start 141.3257 102.2993) (end 141.3257 103.40102) (width 0.2) (layer F.Cu) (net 4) (status 20))
 (segment (start 141.3257 102.2993) (end 141.3257 101.90114) (width 0.25) (layer F.Cu) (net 4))
 (segment (start 141.3257 103.40102) (end 141.3257 101.90114) (width 0.25) (layer F.Cu) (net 4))
 (segment (start 141.3257 100.69746) (end 141.52316 100.5) (width 0.3) (layer F.Cu) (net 4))
 (segment (start 141.3257 101.90114) (end 141.3257 100.69746) (width 0.3) (layer F.Cu) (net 4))
 (segment (start 141.52316 100.5) (end 141.52316 98.95184) (width 0.3) (layer F.Cu) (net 4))
 (segment (start 141.52316 98.95184) (end 144.775 95.7) (width 0.3) (layer F.Cu) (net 4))
 (segment (start 144.775 94.5) (end 144.675 94.4) (width 0.3) (layer F.Cu) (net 4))
 (segment (start 144.775 95.7) (end 144.775 94.5) (width 0.3) (layer F.Cu) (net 4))
 (segment (start 140.82532 103.40102) (end 140.82532 102.95032) (width 0.25) (layer F.Cu) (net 3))
 (segment (start 140.12684 102.25184) (end 140.12684 100.5) (width 0.25) (layer F.Cu) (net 3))
 (segment (start 140.82532 102.95032) (end 140.12684 102.25184) (width 0.25) (layer F.Cu) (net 3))
 (segment (start 140.12684 100.5) (end 140.12684 98.14816) (width 0.3) (layer F.Cu) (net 3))
 (segment (start 142.675 95.6) (end 142.675 94.4) (width 0.3) (layer F.Cu) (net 3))
 (segment (start 140.12684 98.14816) (end 142.675 95.6) (width 0.3) (layer F.Cu) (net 3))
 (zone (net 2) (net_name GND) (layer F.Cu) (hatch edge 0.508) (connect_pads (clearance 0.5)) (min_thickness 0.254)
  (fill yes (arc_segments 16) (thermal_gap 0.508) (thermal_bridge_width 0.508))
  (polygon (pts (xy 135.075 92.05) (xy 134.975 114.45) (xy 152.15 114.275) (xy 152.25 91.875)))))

